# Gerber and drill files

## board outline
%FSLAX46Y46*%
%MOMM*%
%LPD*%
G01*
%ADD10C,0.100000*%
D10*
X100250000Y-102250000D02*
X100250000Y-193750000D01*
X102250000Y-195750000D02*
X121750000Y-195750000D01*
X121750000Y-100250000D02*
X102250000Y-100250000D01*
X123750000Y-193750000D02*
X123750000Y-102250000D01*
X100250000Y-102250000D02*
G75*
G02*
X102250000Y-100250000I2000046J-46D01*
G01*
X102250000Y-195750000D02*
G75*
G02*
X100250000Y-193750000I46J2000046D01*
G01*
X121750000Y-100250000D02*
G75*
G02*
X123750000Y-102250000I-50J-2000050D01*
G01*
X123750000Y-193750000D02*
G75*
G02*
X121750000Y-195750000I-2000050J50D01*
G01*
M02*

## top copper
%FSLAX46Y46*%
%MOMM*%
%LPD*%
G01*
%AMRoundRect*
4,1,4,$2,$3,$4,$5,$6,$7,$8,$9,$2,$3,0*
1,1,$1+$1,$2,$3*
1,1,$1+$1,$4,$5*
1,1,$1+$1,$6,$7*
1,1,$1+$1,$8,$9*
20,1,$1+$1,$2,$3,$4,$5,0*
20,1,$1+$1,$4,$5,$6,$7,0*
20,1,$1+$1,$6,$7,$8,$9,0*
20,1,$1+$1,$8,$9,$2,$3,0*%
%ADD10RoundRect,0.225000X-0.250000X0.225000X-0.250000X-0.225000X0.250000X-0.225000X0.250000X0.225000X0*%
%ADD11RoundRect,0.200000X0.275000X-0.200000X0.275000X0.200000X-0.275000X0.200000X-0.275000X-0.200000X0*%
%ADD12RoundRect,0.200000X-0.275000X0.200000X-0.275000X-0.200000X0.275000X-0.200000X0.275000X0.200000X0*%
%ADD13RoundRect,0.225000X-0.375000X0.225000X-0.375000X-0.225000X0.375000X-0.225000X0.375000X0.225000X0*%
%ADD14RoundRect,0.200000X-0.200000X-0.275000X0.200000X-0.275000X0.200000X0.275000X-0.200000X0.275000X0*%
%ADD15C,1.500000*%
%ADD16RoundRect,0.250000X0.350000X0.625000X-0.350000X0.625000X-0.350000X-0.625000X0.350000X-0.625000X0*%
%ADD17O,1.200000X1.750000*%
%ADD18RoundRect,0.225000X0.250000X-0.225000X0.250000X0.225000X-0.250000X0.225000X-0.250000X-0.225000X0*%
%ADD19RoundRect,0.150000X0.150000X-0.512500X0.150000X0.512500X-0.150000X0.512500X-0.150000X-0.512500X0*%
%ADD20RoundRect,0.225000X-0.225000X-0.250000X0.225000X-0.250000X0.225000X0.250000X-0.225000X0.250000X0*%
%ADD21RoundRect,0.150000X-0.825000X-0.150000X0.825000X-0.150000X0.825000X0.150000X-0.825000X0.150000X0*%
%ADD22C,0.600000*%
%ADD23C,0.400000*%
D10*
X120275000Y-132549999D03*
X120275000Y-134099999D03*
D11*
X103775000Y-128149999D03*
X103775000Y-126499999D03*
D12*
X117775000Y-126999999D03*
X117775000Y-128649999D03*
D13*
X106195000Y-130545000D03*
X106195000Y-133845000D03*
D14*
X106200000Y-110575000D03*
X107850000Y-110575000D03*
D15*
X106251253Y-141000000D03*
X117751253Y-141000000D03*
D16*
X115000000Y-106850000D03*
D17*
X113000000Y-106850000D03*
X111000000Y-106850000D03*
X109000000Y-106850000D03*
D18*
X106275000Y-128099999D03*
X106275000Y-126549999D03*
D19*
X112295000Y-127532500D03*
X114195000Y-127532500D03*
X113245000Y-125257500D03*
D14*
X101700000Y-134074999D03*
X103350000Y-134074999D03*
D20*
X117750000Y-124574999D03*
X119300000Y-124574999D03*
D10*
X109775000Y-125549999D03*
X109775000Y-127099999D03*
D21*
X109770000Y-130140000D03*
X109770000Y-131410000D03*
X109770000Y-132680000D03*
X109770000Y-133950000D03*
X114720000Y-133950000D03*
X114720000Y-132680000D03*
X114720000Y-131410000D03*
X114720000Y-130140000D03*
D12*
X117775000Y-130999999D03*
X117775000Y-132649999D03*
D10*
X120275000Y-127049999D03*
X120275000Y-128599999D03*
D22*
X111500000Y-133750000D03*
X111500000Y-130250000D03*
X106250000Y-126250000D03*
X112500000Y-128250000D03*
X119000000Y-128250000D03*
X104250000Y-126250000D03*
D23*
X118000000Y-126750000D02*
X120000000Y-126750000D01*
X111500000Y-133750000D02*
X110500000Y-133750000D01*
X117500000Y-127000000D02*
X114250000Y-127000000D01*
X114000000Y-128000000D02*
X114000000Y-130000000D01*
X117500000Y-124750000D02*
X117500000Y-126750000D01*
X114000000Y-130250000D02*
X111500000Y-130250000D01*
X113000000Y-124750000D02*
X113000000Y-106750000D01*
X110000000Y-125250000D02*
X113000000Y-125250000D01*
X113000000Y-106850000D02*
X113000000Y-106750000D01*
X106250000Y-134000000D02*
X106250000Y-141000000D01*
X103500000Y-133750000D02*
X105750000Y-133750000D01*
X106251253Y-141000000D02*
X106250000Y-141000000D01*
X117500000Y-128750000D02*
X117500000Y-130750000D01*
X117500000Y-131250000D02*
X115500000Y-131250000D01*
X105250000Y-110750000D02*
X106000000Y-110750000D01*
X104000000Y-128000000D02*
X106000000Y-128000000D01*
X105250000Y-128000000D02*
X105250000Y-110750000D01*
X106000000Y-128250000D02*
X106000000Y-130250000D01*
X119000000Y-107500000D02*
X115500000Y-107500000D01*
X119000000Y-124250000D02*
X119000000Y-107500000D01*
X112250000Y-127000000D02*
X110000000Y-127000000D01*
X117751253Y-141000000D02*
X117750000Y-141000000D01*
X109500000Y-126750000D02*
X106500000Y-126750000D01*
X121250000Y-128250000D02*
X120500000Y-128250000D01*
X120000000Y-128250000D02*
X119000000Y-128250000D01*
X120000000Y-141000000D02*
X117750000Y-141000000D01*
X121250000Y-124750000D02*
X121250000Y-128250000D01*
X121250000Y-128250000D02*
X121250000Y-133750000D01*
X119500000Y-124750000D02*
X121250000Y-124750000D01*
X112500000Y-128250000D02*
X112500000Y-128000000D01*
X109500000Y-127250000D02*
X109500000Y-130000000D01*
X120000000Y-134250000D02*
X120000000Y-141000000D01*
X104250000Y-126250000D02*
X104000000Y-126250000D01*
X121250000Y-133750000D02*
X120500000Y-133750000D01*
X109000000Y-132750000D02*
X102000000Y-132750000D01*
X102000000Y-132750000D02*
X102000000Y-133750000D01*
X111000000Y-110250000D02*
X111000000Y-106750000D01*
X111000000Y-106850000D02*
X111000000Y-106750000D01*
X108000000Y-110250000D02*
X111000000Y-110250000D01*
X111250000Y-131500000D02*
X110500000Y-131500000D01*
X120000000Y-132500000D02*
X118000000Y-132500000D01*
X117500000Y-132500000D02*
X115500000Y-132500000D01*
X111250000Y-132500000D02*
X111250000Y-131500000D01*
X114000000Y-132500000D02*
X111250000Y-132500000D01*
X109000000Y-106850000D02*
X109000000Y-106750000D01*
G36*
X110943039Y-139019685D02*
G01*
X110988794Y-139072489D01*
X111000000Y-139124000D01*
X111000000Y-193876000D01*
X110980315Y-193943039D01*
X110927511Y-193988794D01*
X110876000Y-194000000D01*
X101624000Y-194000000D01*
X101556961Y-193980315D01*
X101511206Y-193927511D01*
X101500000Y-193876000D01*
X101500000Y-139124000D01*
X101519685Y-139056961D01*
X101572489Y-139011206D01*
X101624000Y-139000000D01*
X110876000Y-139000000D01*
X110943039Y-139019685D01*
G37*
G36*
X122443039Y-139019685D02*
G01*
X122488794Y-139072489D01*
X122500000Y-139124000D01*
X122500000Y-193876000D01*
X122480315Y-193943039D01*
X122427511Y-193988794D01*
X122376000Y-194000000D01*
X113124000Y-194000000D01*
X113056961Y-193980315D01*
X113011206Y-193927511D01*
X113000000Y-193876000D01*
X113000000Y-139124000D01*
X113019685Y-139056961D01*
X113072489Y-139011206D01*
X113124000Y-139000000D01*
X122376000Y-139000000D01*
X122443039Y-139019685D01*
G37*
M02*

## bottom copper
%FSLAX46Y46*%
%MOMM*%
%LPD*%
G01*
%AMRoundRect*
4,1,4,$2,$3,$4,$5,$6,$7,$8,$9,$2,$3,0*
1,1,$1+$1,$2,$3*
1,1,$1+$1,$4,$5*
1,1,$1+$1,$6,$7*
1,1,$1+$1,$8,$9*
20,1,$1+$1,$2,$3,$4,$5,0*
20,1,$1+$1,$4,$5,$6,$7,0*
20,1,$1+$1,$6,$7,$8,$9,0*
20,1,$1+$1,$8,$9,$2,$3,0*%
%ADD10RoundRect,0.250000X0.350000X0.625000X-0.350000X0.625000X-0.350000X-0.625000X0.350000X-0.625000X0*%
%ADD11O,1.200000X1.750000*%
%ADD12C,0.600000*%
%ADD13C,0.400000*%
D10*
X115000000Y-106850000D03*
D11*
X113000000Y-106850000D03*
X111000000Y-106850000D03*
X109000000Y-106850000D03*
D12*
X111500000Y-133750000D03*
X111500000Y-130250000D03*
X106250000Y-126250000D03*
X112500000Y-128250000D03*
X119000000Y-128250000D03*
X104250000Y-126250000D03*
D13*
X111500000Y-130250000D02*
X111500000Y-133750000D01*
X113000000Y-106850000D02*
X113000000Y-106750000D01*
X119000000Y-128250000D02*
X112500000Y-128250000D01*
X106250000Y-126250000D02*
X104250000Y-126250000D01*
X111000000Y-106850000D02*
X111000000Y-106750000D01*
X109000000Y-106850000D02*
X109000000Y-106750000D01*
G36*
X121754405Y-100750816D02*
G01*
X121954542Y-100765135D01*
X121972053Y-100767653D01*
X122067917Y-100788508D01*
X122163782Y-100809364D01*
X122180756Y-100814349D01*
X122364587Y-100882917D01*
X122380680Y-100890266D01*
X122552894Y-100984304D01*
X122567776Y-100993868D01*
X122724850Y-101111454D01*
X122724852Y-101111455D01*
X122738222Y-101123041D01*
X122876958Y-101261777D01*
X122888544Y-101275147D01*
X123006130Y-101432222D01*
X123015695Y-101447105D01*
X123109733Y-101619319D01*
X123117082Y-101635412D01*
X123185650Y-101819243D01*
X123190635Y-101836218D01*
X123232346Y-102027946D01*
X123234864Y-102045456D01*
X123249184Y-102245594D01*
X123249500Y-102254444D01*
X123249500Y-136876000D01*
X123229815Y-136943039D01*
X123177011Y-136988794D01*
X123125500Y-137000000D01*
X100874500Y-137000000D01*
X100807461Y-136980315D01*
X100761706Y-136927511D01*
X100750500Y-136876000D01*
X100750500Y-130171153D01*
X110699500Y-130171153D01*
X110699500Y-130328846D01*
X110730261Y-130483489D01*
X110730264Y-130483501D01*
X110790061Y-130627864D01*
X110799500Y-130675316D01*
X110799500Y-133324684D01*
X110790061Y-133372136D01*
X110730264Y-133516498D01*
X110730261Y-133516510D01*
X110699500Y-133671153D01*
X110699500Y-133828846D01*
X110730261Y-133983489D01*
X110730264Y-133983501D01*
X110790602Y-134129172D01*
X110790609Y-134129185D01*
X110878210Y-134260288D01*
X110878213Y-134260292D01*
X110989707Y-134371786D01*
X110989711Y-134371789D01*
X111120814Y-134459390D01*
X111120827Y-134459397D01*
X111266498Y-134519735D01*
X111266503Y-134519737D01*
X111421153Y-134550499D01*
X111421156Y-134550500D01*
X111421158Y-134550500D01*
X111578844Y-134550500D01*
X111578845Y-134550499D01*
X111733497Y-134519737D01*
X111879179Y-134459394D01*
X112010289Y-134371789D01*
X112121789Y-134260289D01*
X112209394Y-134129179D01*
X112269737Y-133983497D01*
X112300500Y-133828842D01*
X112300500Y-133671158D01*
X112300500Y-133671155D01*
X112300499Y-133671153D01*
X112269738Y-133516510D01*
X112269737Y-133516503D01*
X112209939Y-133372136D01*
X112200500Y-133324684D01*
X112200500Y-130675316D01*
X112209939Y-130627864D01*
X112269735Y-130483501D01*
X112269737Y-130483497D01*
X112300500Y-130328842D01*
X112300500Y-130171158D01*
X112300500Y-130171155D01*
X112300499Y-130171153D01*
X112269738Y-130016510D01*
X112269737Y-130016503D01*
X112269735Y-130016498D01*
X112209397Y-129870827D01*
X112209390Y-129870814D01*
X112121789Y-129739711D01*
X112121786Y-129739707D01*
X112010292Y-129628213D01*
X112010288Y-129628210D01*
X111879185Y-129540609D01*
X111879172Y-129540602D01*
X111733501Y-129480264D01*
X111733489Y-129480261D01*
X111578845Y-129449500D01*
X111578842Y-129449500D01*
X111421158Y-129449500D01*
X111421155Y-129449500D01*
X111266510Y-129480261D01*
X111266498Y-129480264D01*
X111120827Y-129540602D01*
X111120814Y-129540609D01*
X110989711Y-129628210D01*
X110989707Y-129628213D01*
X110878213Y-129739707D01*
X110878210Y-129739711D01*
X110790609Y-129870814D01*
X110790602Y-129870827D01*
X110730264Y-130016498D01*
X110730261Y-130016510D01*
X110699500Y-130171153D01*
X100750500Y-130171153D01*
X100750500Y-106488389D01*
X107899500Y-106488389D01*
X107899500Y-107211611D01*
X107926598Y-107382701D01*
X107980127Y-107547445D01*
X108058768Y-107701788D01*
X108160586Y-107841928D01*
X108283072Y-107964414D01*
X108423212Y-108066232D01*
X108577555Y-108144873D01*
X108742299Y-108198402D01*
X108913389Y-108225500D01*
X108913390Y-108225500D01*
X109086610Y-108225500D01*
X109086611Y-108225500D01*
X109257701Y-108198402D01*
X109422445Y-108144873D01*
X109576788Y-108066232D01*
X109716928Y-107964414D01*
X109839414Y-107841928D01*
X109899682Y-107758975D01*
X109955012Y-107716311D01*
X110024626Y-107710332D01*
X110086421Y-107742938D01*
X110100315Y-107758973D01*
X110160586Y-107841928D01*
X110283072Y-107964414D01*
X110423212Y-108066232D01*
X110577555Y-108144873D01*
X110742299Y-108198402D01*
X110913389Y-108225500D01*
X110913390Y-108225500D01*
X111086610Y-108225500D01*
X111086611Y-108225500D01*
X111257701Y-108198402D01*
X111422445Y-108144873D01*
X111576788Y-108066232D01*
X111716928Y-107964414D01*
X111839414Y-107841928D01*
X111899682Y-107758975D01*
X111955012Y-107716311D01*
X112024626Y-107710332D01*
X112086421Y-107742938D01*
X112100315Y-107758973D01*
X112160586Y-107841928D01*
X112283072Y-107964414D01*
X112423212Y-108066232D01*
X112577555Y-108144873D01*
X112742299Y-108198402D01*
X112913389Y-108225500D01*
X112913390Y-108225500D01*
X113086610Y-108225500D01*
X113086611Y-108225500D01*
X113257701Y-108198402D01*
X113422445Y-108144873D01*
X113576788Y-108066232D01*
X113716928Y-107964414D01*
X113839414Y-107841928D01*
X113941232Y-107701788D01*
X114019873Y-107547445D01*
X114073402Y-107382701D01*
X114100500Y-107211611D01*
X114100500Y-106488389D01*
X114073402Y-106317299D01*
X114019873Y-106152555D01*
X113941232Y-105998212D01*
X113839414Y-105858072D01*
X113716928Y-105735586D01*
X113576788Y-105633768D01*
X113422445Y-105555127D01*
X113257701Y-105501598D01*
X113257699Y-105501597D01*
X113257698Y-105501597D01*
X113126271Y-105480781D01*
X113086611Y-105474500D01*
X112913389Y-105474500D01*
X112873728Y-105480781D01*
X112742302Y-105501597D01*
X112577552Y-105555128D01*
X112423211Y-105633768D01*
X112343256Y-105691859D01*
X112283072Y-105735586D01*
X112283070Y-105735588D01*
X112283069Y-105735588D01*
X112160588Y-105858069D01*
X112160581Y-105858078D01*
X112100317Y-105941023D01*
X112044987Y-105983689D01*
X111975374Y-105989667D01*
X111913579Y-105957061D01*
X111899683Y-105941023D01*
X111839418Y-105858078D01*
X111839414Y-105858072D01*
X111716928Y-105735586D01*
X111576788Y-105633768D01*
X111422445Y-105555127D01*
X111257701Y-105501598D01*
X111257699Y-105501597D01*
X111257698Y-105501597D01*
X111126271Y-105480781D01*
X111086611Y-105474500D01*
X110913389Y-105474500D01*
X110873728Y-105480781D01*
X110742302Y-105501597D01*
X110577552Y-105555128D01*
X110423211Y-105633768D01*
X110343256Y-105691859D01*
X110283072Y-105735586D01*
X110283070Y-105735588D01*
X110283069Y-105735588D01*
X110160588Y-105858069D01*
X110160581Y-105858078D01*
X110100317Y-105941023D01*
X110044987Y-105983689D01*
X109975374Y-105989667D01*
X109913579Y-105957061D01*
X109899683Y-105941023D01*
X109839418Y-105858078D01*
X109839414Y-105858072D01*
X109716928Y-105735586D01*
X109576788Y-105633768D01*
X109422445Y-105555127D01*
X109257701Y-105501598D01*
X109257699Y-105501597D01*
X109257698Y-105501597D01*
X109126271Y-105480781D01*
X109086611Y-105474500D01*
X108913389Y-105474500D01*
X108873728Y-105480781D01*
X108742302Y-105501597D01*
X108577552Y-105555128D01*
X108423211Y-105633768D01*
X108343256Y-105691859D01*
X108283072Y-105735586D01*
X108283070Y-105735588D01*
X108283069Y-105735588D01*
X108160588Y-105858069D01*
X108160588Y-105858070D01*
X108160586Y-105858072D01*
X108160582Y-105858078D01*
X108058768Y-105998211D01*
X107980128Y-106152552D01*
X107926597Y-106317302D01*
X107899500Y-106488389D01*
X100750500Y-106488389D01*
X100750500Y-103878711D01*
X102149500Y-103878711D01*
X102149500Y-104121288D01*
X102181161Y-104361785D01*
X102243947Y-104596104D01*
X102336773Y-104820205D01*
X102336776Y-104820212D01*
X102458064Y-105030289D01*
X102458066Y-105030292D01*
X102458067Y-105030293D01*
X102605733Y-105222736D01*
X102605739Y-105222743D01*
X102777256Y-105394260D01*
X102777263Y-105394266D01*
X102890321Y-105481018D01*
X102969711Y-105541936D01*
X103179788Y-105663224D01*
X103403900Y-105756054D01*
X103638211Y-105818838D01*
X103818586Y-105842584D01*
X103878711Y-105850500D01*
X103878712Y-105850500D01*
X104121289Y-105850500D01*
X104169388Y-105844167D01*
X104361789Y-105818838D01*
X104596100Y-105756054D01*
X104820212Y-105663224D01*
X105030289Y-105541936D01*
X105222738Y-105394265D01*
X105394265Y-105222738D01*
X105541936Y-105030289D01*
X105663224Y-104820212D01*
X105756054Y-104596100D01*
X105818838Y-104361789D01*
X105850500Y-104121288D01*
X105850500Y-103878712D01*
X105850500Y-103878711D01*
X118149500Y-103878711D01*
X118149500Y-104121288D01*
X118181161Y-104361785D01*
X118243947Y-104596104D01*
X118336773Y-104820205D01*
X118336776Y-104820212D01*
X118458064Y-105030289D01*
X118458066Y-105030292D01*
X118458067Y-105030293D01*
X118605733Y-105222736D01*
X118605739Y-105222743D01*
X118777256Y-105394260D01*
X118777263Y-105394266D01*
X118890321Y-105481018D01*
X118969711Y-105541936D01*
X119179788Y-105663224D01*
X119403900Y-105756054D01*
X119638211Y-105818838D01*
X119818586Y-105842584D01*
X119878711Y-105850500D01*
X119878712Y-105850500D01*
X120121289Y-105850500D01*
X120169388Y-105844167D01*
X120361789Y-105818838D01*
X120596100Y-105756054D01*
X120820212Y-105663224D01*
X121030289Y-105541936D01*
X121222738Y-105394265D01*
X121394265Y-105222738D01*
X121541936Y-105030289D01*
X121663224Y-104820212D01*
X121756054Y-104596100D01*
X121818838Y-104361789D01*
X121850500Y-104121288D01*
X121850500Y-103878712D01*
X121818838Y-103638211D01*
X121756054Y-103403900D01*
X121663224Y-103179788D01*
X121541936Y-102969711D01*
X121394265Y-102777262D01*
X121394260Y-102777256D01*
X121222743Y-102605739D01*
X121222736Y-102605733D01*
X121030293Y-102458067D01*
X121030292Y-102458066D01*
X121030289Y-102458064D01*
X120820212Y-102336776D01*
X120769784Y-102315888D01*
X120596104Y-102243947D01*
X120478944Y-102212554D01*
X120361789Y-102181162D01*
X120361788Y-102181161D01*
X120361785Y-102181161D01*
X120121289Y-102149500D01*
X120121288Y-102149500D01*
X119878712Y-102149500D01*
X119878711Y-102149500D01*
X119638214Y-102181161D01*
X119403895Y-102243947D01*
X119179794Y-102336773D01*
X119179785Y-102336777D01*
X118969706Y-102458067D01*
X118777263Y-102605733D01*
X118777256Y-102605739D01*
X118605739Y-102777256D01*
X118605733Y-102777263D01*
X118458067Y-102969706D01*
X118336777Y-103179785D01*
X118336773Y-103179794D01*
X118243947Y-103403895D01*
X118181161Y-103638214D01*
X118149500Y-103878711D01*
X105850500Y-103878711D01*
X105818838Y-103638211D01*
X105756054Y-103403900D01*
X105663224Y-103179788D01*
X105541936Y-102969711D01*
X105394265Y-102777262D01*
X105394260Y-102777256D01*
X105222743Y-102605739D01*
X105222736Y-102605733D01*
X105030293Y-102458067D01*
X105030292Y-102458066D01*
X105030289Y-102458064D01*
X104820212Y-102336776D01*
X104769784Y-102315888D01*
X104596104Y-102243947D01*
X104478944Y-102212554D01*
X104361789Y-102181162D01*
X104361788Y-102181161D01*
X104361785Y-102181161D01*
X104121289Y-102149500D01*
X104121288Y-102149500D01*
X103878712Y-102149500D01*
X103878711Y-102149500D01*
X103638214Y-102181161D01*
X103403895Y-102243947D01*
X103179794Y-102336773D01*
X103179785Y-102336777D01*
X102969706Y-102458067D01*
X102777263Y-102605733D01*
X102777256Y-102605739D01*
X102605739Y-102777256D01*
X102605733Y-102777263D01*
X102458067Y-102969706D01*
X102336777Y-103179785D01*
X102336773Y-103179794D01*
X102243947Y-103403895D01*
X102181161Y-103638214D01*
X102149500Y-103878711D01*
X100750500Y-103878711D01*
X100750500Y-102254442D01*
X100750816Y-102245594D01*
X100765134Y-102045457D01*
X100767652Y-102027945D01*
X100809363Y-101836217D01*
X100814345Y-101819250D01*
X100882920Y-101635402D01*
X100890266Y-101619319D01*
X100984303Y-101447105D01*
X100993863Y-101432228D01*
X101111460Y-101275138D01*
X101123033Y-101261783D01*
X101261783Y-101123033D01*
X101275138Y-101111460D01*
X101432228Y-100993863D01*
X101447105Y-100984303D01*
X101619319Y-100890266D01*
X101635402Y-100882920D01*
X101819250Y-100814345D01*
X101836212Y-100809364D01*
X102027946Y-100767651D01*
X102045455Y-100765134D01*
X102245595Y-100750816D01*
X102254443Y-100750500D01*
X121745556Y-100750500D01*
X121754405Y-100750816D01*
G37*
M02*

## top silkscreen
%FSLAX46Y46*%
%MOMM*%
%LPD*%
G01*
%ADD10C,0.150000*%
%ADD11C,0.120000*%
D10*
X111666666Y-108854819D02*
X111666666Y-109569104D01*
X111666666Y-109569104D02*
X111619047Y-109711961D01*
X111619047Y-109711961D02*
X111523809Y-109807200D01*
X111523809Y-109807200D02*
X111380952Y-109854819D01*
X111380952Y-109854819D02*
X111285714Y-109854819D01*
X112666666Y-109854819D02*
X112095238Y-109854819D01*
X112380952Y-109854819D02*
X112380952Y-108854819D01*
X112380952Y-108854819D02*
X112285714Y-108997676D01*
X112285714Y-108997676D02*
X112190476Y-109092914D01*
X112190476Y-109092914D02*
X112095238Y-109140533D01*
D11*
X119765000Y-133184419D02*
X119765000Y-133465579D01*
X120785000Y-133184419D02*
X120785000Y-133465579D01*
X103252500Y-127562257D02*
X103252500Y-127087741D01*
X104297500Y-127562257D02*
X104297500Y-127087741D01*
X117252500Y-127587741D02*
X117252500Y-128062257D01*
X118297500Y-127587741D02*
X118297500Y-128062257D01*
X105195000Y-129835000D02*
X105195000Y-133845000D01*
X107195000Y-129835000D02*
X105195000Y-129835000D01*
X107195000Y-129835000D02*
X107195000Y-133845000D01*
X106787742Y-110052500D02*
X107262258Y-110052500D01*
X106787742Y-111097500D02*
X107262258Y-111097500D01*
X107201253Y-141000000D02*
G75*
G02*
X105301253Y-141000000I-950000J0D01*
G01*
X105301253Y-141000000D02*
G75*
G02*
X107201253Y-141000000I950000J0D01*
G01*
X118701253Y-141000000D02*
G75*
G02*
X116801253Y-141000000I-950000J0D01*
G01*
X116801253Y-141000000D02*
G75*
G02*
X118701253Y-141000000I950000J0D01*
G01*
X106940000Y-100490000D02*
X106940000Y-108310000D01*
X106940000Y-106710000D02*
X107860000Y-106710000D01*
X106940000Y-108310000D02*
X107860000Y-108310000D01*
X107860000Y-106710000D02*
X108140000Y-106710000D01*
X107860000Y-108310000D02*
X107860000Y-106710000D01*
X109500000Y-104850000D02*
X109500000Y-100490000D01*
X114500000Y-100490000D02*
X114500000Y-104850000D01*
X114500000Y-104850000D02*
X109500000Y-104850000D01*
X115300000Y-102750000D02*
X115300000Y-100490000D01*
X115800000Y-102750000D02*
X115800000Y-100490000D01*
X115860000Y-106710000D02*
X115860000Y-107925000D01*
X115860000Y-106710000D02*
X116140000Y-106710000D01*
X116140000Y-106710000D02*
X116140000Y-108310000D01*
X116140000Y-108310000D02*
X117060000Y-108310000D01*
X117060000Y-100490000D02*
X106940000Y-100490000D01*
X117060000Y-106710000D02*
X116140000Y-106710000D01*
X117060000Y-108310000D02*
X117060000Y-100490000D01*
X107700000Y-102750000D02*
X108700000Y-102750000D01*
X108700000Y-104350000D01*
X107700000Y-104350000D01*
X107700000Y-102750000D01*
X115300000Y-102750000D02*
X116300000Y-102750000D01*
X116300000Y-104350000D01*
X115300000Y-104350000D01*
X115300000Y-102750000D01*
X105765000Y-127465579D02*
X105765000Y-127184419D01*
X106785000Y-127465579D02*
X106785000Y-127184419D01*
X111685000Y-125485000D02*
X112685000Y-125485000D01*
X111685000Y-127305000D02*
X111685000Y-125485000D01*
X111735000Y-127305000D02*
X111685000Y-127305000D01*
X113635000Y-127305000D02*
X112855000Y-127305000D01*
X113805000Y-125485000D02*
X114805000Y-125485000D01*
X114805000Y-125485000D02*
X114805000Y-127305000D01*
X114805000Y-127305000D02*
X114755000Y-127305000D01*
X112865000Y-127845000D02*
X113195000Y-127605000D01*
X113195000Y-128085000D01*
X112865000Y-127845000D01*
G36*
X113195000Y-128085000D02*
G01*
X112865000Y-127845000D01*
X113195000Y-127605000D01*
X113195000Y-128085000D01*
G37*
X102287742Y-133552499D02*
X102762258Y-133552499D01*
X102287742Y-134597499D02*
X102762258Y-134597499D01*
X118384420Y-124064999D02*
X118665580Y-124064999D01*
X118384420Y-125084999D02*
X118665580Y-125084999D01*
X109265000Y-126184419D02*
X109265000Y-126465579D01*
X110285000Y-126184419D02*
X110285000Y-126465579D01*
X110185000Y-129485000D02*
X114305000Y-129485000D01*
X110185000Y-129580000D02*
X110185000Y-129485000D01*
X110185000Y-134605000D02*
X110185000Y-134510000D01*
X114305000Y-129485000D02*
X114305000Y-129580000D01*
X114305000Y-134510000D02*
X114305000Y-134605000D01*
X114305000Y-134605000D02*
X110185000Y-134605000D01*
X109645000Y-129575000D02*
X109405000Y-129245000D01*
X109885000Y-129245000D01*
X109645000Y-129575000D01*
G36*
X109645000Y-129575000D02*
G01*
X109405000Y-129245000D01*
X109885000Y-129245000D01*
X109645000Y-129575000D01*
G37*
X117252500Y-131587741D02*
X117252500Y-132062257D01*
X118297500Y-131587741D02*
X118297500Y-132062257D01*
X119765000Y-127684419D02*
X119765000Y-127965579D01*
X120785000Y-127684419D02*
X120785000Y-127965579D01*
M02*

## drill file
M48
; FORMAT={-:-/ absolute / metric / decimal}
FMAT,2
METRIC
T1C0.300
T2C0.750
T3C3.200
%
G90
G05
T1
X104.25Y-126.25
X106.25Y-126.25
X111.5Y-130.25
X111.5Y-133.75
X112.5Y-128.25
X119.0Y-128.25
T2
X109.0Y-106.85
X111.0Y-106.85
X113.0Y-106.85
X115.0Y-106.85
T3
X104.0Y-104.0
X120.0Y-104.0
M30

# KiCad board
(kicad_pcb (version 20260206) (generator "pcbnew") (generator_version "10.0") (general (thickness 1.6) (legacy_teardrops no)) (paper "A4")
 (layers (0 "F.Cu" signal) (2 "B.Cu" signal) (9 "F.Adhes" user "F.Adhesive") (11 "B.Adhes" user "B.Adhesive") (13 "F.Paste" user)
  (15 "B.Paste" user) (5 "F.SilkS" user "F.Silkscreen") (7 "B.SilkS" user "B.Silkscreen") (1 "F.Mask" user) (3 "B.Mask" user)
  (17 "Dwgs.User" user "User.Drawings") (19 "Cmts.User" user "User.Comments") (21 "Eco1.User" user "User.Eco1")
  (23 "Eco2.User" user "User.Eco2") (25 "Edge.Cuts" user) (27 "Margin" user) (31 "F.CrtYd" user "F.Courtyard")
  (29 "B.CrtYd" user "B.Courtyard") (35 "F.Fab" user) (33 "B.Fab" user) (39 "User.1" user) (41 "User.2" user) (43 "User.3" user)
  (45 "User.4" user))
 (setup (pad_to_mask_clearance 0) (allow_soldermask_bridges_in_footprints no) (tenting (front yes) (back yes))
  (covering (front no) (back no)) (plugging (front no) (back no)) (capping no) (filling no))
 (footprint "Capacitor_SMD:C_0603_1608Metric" (layer "F.Cu") (at 120.275 133.324999 -90)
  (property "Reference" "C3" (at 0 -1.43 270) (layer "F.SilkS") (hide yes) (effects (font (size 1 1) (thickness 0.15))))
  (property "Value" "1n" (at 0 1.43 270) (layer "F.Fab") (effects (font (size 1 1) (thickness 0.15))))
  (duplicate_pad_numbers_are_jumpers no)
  (fp_line (start -0.14058 0.51) (end 0.14058 0.51) (stroke (width 0.12) (type solid)) (layer "F.SilkS"))
  (fp_line (start -0.14058 -0.51) (end 0.14058 -0.51) (stroke (width 0.12) (type solid)) (layer "F.SilkS"))
  (pad "1" smd roundrect (at -0.775 0 270) (size 0.9 0.95) (layers "F.Cu" "F.Mask" "F.Paste") (roundrect_rratio 0.25) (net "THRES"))
  (pad "2" smd roundrect (at 0.775 0 270) (size 0.9 0.95) (layers "F.Cu" "F.Mask" "F.Paste") (roundrect_rratio 0.25) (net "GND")))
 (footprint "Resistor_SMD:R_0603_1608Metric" (layer "F.Cu") (at 103.775 127.324999 90)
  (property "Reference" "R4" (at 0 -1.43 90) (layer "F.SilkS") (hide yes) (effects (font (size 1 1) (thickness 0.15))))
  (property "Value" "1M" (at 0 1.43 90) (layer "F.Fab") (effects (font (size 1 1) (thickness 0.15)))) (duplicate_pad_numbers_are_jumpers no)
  (fp_line (start -0.237258 -0.5225) (end 0.237258 -0.5225) (stroke (width 0.12) (type solid)) (layer "F.SilkS"))
  (fp_line (start -0.237258 0.5225) (end 0.237258 0.5225) (stroke (width 0.12) (type solid)) (layer "F.SilkS"))
  (pad "1" smd roundrect (at -0.825 0 90) (size 0.8 0.95) (layers "F.Cu" "F.Mask" "F.Paste") (roundrect_rratio 0.25) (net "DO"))
  (pad "2" smd roundrect (at 0.825 0 90) (size 0.8 0.95) (layers "F.Cu" "F.Mask" "F.Paste") (roundrect_rratio 0.25) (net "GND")))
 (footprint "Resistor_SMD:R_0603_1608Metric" (layer "F.Cu") (at 117.775 127.824999 -90)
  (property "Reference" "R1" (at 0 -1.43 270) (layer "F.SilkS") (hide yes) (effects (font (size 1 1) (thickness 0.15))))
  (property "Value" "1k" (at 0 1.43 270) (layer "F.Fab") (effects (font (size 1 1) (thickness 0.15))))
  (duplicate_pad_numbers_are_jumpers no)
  (fp_line (start -0.237258 0.5225) (end 0.237258 0.5225) (stroke (width 0.12) (type solid)) (layer "F.SilkS"))
  (fp_line (start -0.237258 -0.5225) (end 0.237258 -0.5225) (stroke (width 0.12) (type solid)) (layer "F.SilkS"))
  (pad "1" smd roundrect (at -0.825 0 270) (size 0.8 0.95) (layers "F.Cu" "F.Mask" "F.Paste") (roundrect_rratio 0.25) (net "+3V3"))
  (pad "2" smd roundrect (at 0.825 0 270) (size 0.8 0.95) (layers "F.Cu" "F.Mask" "F.Paste") (roundrect_rratio 0.25) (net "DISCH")))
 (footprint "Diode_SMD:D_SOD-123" (layer "F.Cu") (at 106.195 132.195 -90)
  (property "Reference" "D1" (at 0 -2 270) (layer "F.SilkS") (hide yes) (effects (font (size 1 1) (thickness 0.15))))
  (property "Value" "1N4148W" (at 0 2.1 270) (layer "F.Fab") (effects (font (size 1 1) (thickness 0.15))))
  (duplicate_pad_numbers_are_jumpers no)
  (fp_line (start -2.36 1) (end 1.65 1) (stroke (width 0.12) (type solid)) (layer "F.SilkS"))
  (fp_line (start -2.36 -1) (end -2.36 1) (stroke (width 0.12) (type solid)) (layer "F.SilkS"))
  (fp_line (start -2.36 -1) (end 1.65 -1) (stroke (width 0.12) (type solid)) (layer "F.SilkS"))
  (pad "1" smd roundrect (at -1.65 0 270) (size 0.9 1.2) (layers "F.Cu" "F.Mask" "F.Paste") (roundrect_rratio 0.25) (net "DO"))
  (pad "2" smd roundrect (at 1.65 0 270) (size 0.9 1.2) (layers "F.Cu" "F.Mask" "F.Paste") (roundrect_rratio 0.25) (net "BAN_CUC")))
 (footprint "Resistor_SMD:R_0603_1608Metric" (layer "F.Cu") (at 107.025 110.575)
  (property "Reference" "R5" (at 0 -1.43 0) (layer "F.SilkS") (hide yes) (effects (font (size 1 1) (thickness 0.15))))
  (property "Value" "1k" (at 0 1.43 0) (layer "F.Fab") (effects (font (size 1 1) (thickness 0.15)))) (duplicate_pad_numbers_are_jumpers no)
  (fp_line (start -0.237258 -0.5225) (end 0.237258 -0.5225) (stroke (width 0.12) (type solid)) (layer "F.SilkS"))
  (fp_line (start -0.237258 0.5225) (end 0.237258 0.5225) (stroke (width 0.12) (type solid)) (layer "F.SilkS"))
  (pad "1" smd roundrect (at -0.825 0) (size 0.8 0.95) (layers "F.Cu" "F.Mask" "F.Paste") (roundrect_rratio 0.25) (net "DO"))
  (pad "2" smd roundrect (at 0.825 0) (size 0.8 0.95) (layers "F.Cu" "F.Mask" "F.Paste") (roundrect_rratio 0.25) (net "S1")))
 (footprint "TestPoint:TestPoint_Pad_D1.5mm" (layer "F.Cu") (at 106.251253 141)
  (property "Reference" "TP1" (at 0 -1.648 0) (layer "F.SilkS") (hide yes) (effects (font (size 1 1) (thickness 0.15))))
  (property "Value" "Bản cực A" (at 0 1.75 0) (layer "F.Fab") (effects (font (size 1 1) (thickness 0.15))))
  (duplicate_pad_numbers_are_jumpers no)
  (fp_circle (center 0 0) (end 0 0.95) (stroke (width 0.12) (type solid)) (fill no) (layer "F.SilkS"))
  (pad "1" smd circle (at 0 0) (size 1.5 1.5) (layers "F.Cu" "F.Mask") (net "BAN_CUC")))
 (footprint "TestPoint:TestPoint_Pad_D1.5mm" (layer "F.Cu") (at 117.751253 141)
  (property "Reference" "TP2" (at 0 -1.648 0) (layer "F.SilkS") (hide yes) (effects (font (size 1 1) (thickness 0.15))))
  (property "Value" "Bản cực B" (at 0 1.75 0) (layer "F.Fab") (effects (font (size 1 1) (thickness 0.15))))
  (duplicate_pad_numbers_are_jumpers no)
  (fp_circle (center 0 0) (end 0 0.95) (stroke (width 0.12) (type solid)) (fill no) (layer "F.SilkS"))
  (pad "1" smd circle (at 0 0) (size 1.5 1.5) (layers "F.Cu" "F.Mask") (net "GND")))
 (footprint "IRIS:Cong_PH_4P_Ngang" (layer "F.Cu") (at 115 106.85 180)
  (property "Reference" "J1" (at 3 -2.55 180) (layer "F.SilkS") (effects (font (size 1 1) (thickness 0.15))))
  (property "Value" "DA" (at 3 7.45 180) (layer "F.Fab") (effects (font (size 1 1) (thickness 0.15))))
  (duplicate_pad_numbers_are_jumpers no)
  (fp_line (start 8.06 6.36) (end 8.06 -1.46) (stroke (width 0.12) (type solid)) (layer "F.SilkS"))
  (fp_line (start 8.06 0.14) (end 7.14 0.14) (stroke (width 0.12) (type solid)) (layer "F.SilkS"))
  (fp_line (start 8.06 -1.46) (end 7.14 -1.46) (stroke (width 0.12) (type solid)) (layer "F.SilkS"))
  (fp_line (start 7.14 0.14) (end 6.86 0.14) (stroke (width 0.12) (type solid)) (layer "F.SilkS"))
  (fp_line (start 7.14 -1.46) (end 7.14 0.14) (stroke (width 0.12) (type solid)) (layer "F.SilkS"))
  (fp_line (start 5.5 2) (end 5.5 6.36) (stroke (width 0.12) (type solid)) (layer "F.SilkS"))
  (fp_line (start 0.5 6.36) (end 0.5 2) (stroke (width 0.12) (type solid)) (layer "F.SilkS"))
  (fp_line (start 0.5 2) (end 5.5 2) (stroke (width 0.12) (type solid)) (layer "F.SilkS"))
  (fp_line (start -0.3 4.1) (end -0.3 6.36) (stroke (width 0.12) (type solid)) (layer "F.SilkS"))
  (fp_line (start -0.8 4.1) (end -0.8 6.36) (stroke (width 0.12) (type solid)) (layer "F.SilkS"))
  (fp_line (start -0.86 0.14) (end -0.86 -1.075) (stroke (width 0.12) (type solid)) (layer "F.SilkS"))
  (fp_line (start -0.86 0.14) (end -1.14 0.14) (stroke (width 0.12) (type solid)) (layer "F.SilkS"))
  (fp_line (start -1.14 0.14) (end -1.14 -1.46) (stroke (width 0.12) (type solid)) (layer "F.SilkS"))
  (fp_line (start -1.14 -1.46) (end -2.06 -1.46) (stroke (width 0.12) (type solid)) (layer "F.SilkS"))
  (fp_line (start -2.06 6.36) (end 8.06 6.36) (stroke (width 0.12) (type solid)) (layer "F.SilkS"))
  (fp_line (start -2.06 0.14) (end -1.14 0.14) (stroke (width 0.12) (type solid)) (layer "F.SilkS"))
  (fp_line (start -2.06 -1.46) (end -2.06 6.36) (stroke (width 0.12) (type solid)) (layer "F.SilkS"))
  (fp_rect (start 6.3 2.5) (end 7.3 4.1) (stroke (width 0.12) (type solid)) (fill no) (layer "F.SilkS"))
  (fp_rect (start -1.3 2.5) (end -0.3 4.1) (stroke (width 0.12) (type solid)) (fill no) (layer "F.SilkS"))
  (pad "1" thru_hole roundrect (at 0 0 180) (size 1.2 1.75) (drill 0.75) (layers "*.Cu" "*.Mask") (remove_unused_layers no)
   (roundrect_rratio 0.208333) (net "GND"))
  (pad "2" thru_hole oval (at 2 0 180) (size 1.2 1.75) (drill 0.75) (layers "*.Cu" "*.Mask") (remove_unused_layers no) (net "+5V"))
  (pad "3" thru_hole oval (at 4 0 180) (size 1.2 1.75) (drill 0.75) (layers "*.Cu" "*.Mask") (remove_unused_layers no) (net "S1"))
  (pad "4" thru_hole oval (at 6 0 180) (size 1.2 1.75) (drill 0.75) (layers "*.Cu" "*.Mask") (remove_unused_layers no)
   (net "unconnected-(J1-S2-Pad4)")))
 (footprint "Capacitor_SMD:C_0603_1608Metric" (layer "F.Cu") (at 106.275 127.324999 90)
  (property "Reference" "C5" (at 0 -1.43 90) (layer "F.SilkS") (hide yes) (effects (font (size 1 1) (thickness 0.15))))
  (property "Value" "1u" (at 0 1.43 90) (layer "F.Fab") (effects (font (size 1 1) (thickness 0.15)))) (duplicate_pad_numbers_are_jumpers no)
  (fp_line (start -0.14058 -0.51) (end 0.14058 -0.51) (stroke (width 0.12) (type solid)) (layer "F.SilkS"))
  (fp_line (start -0.14058 0.51) (end 0.14058 0.51) (stroke (width 0.12) (type solid)) (layer "F.SilkS"))
  (pad "1" smd roundrect (at -0.775 0 90) (size 0.9 0.95) (layers "F.Cu" "F.Mask" "F.Paste") (roundrect_rratio 0.25) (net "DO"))
  (pad "2" smd roundrect (at 0.775 0 90) (size 0.9 0.95) (layers "F.Cu" "F.Mask" "F.Paste") (roundrect_rratio 0.25) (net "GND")))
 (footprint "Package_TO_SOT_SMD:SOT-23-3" (layer "F.Cu") (at 113.245 126.395 90)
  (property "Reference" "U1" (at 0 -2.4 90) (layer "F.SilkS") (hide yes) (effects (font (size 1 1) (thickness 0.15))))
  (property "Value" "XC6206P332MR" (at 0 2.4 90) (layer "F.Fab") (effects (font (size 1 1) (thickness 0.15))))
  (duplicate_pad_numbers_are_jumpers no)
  (fp_line (start 0.91 -1.56) (end 0.91 -0.56) (stroke (width 0.12) (type solid)) (layer "F.SilkS"))
  (fp_line (start -0.91 -1.56) (end 0.91 -1.56) (stroke (width 0.12) (type solid)) (layer "F.SilkS"))
  (fp_line (start -0.91 -1.51) (end -0.91 -1.56) (stroke (width 0.12) (type solid)) (layer "F.SilkS"))
  (fp_line (start -0.91 0.39) (end -0.91 -0.39) (stroke (width 0.12) (type solid)) (layer "F.SilkS"))
  (fp_line (start 0.91 0.56) (end 0.91 1.56) (stroke (width 0.12) (type solid)) (layer "F.SilkS"))
  (fp_line (start 0.91 1.56) (end -0.91 1.56) (stroke (width 0.12) (type solid)) (layer "F.SilkS"))
  (fp_line (start -0.91 1.56) (end -0.91 1.51) (stroke (width 0.12) (type solid)) (layer "F.SilkS"))
  (fp_poly (pts (xy -1.45 -0.38) (xy -1.21 -0.05) (xy -1.69 -0.05)) (stroke (width 0.12) (type solid)) (fill yes) (layer "F.SilkS"))
  (pad "1" smd roundrect (at -1.1375 -0.95 90) (size 1.325 0.6) (layers "F.Cu" "F.Mask" "F.Paste") (roundrect_rratio 0.25) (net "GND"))
  (pad "2" smd roundrect (at -1.1375 0.95 90) (size 1.325 0.6) (layers "F.Cu" "F.Mask" "F.Paste") (roundrect_rratio 0.25) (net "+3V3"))
  (pad "3" smd roundrect (at 1.1375 0 90) (size 1.325 0.6) (layers "F.Cu" "F.Mask" "F.Paste") (roundrect_rratio 0.25) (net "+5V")))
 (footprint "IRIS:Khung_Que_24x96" (layer "F.Cu") (at 100 196)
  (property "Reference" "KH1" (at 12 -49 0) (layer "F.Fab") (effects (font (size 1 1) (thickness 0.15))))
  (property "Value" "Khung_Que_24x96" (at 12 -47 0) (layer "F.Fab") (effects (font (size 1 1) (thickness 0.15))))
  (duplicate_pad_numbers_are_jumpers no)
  (fp_line (start 0.25 -93.75) (end 0.25 -2.25) (stroke (width 0.1) (type solid)) (layer "Edge.Cuts"))
  (fp_line (start 2.25 -0.25) (end 21.75 -0.25) (stroke (width 0.1) (type solid)) (layer "Edge.Cuts"))
  (fp_line (start 21.75 -95.75) (end 2.25 -95.75) (stroke (width 0.1) (type solid)) (layer "Edge.Cuts"))
  (fp_line (start 23.75 -2.25) (end 23.75 -93.75) (stroke (width 0.1) (type solid)) (layer "Edge.Cuts"))
  (fp_arc (start 0.25 -93.75) (mid 0.8358 -95.1642) (end 2.25 -95.75) (stroke (width 0.1) (type solid)) (layer "Edge.Cuts"))
  (fp_arc (start 2.25 -0.25) (mid 0.8358 -0.8358) (end 0.25 -2.25) (stroke (width 0.1) (type solid)) (layer "Edge.Cuts"))
  (fp_arc (start 21.75 -95.75) (mid 23.164199 -95.164199) (end 23.75 -93.75) (stroke (width 0.1) (type solid)) (layer "Edge.Cuts"))
  (fp_arc (start 23.75 -2.25) (mid 23.164199 -0.835801) (end 21.75 -0.25) (stroke (width 0.1) (type solid)) (layer "Edge.Cuts"))
  (pad "" np_thru_hole circle (at 4 -92) (size 3.2 3.2) (drill 3.2) (layers "*.Cu" "*.Mask"))
  (pad "" np_thru_hole circle (at 20 -92) (size 3.2 3.2) (drill 3.2) (layers "*.Cu" "*.Mask")))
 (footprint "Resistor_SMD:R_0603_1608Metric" (layer "F.Cu") (at 102.525 134.074999)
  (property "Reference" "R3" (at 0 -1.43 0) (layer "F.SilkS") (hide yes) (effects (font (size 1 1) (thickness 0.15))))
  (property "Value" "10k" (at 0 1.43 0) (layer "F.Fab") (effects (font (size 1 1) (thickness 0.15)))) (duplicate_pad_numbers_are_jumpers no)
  (fp_line (start -0.237258 -0.5225) (end 0.237258 -0.5225) (stroke (width 0.12) (type solid)) (layer "F.SilkS"))
  (fp_line (start -0.237258 0.5225) (end 0.237258 0.5225) (stroke (width 0.12) (type solid)) (layer "F.SilkS"))
  (pad "1" smd roundrect (at -0.825 0) (size 0.8 0.95) (layers "F.Cu" "F.Mask" "F.Paste") (roundrect_rratio 0.25) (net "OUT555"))
  (pad "2" smd roundrect (at 0.825 0) (size 0.8 0.95) (layers "F.Cu" "F.Mask" "F.Paste") (roundrect_rratio 0.25) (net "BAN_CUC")))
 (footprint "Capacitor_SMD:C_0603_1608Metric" (layer "F.Cu") (at 118.525 124.574999)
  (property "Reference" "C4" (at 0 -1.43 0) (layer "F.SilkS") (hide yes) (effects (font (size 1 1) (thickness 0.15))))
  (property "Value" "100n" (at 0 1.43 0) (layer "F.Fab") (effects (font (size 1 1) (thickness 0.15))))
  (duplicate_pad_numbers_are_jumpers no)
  (fp_line (start -0.14058 -0.51) (end 0.14058 -0.51) (stroke (width 0.12) (type solid)) (layer "F.SilkS"))
  (fp_line (start -0.14058 0.51) (end 0.14058 0.51) (stroke (width 0.12) (type solid)) (layer "F.SilkS"))
  (pad "1" smd roundrect (at -0.775 0) (size 0.9 0.95) (layers "F.Cu" "F.Mask" "F.Paste") (roundrect_rratio 0.25) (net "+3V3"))
  (pad "2" smd roundrect (at 0.775 0) (size 0.9 0.95) (layers "F.Cu" "F.Mask" "F.Paste") (roundrect_rratio 0.25) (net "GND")))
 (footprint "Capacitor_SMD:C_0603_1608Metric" (layer "F.Cu") (at 109.775 126.324999 -90)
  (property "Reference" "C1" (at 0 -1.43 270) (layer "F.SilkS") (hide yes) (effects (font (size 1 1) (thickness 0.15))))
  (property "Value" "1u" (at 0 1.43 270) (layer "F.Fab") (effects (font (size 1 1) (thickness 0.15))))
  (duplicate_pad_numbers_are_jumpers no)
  (fp_line (start -0.14058 0.51) (end 0.14058 0.51) (stroke (width 0.12) (type solid)) (layer "F.SilkS"))
  (fp_line (start -0.14058 -0.51) (end 0.14058 -0.51) (stroke (width 0.12) (type solid)) (layer "F.SilkS"))
  (pad "1" smd roundrect (at -0.775 0 270) (size 0.9 0.95) (layers "F.Cu" "F.Mask" "F.Paste") (roundrect_rratio 0.25) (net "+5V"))
  (pad "2" smd roundrect (at 0.775 0 270) (size 0.9 0.95) (layers "F.Cu" "F.Mask" "F.Paste") (roundrect_rratio 0.25) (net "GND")))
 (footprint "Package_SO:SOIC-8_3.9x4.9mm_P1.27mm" (layer "F.Cu") (at 112.245 132.045)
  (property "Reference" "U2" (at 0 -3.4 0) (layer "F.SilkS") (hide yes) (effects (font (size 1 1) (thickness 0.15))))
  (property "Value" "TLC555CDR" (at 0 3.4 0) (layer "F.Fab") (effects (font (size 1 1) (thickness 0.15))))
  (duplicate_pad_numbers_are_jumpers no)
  (fp_line (start -2.06 -2.56) (end 2.06 -2.56) (stroke (width 0.12) (type solid)) (layer "F.SilkS"))
  (fp_line (start -2.06 -2.465) (end -2.06 -2.56) (stroke (width 0.12) (type solid)) (layer "F.SilkS"))
  (fp_line (start -2.06 2.56) (end -2.06 2.465) (stroke (width 0.12) (type solid)) (layer "F.SilkS"))
  (fp_line (start 2.06 -2.56) (end 2.06 -2.465) (stroke (width 0.12) (type solid)) (layer "F.SilkS"))
  (fp_line (start 2.06 2.465) (end 2.06 2.56) (stroke (width 0.12) (type solid)) (layer "F.SilkS"))
  (fp_line (start 2.06 2.56) (end -2.06 2.56) (stroke (width 0.12) (type solid)) (layer "F.SilkS"))
  (fp_poly (pts (xy -2.6 -2.47) (xy -2.84 -2.8) (xy -2.36 -2.8)) (stroke (width 0.12) (type solid)) (fill yes) (layer "F.SilkS"))
  (pad "1" smd roundrect (at -2.475 -1.905) (size 1.95 0.6) (layers "F.Cu" "F.Mask" "F.Paste") (roundrect_rratio 0.25) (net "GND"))
  (pad "2" smd roundrect (at -2.475 -0.635) (size 1.95 0.6) (layers "F.Cu" "F.Mask" "F.Paste") (roundrect_rratio 0.25) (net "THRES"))
  (pad "3" smd roundrect (at -2.475 0.635) (size 1.95 0.6) (layers "F.Cu" "F.Mask" "F.Paste") (roundrect_rratio 0.25) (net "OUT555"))
  (pad "4" smd roundrect (at -2.475 1.905) (size 1.95 0.6) (layers "F.Cu" "F.Mask" "F.Paste") (roundrect_rratio 0.25) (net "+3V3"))
  (pad "5" smd roundrect (at 2.475 1.905) (size 1.95 0.6) (layers "F.Cu" "F.Mask" "F.Paste") (roundrect_rratio 0.25)
   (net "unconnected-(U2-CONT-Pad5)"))
  (pad "6" smd roundrect (at 2.475 0.635) (size 1.95 0.6) (layers "F.Cu" "F.Mask" "F.Paste") (roundrect_rratio 0.25) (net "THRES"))
  (pad "7" smd roundrect (at 2.475 -0.635) (size 1.95 0.6) (layers "F.Cu" "F.Mask" "F.Paste") (roundrect_rratio 0.25) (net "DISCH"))
  (pad "8" smd roundrect (at 2.475 -1.905) (size 1.95 0.6) (layers "F.Cu" "F.Mask" "F.Paste") (roundrect_rratio 0.25) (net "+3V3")))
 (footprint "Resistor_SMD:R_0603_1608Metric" (layer "F.Cu") (at 117.775 131.824999 -90)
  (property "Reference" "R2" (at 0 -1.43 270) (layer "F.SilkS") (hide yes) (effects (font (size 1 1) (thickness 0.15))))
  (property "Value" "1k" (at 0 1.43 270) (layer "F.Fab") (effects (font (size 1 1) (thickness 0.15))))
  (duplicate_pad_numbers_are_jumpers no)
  (fp_line (start -0.237258 0.5225) (end 0.237258 0.5225) (stroke (width 0.12) (type solid)) (layer "F.SilkS"))
  (fp_line (start -0.237258 -0.5225) (end 0.237258 -0.5225) (stroke (width 0.12) (type solid)) (layer "F.SilkS"))
  (pad "1" smd roundrect (at -0.825 0 270) (size 0.8 0.95) (layers "F.Cu" "F.Mask" "F.Paste") (roundrect_rratio 0.25) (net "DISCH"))
  (pad "2" smd roundrect (at 0.825 0 270) (size 0.8 0.95) (layers "F.Cu" "F.Mask" "F.Paste") (roundrect_rratio 0.25) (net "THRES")))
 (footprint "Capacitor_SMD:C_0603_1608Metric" (layer "F.Cu") (at 120.275 127.824999 -90)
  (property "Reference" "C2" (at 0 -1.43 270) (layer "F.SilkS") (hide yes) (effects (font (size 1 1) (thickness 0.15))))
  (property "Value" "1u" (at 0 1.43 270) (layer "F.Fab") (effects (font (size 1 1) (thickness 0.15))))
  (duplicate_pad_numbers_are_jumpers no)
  (fp_line (start -0.14058 0.51) (end 0.14058 0.51) (stroke (width 0.12) (type solid)) (layer "F.SilkS"))
  (fp_line (start -0.14058 -0.51) (end 0.14058 -0.51) (stroke (width 0.12) (type solid)) (layer "F.SilkS"))
  (pad "1" smd roundrect (at -0.775 0 270) (size 0.9 0.95) (layers "F.Cu" "F.Mask" "F.Paste") (roundrect_rratio 0.25) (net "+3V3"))
  (pad "2" smd roundrect (at 0.775 0 270) (size 0.9 0.95) (layers "F.Cu" "F.Mask" "F.Paste") (roundrect_rratio 0.25) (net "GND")))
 (segment (start 118 126.75) (end 120 126.75) (width 0.4) (layer "F.Cu") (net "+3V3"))
 (segment (start 111.5 133.75) (end 110.5 133.75) (width 0.4) (layer "F.Cu") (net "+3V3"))
 (segment (start 117.5 127) (end 114.25 127) (width 0.4) (layer "F.Cu") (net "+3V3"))
 (segment (start 114 128) (end 114 130) (width 0.4) (layer "F.Cu") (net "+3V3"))
 (segment (start 117.5 124.75) (end 117.5 126.75) (width 0.4) (layer "F.Cu") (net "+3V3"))
 (segment (start 114 130.25) (end 111.5 130.25) (width 0.4) (layer "F.Cu") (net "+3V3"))
 (via (at 111.5 133.75) (size 0.6) (drill 0.3) (layers "F.Cu" "B.Cu") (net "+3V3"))
 (via (at 111.5 130.25) (size 0.6) (drill 0.3) (layers "F.Cu" "B.Cu") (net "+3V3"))
 (segment (start 111.5 130.25) (end 111.5 133.75) (width 0.4) (layer "B.Cu") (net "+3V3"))
 (segment (start 113 124.75) (end 113 106.75) (width 0.4) (layer "F.Cu") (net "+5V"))
 (segment (start 110 125.25) (end 113 125.25) (width 0.4) (layer "F.Cu") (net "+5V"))
 (segment (start 113 106.85) (end 113 106.75) (width 0.4) (layer "F.Cu") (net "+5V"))
 (segment (start 113 106.85) (end 113 106.75) (width 0.4) (layer "B.Cu") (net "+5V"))
 (segment (start 106.25 134) (end 106.25 141) (width 0.4) (layer "F.Cu") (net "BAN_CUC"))
 (segment (start 103.5 133.75) (end 105.75 133.75) (width 0.4) (layer "F.Cu") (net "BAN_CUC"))
 (segment (start 106.251253 141) (end 106.25 141) (width 0.4) (layer "F.Cu") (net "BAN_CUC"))
 (segment (start 117.5 128.75) (end 117.5 130.75) (width 0.4) (layer "F.Cu") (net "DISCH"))
 (segment (start 117.5 131.25) (end 115.5 131.25) (width 0.4) (layer "F.Cu") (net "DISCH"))
 (segment (start 105.25 110.75) (end 106 110.75) (width 0.4) (layer "F.Cu") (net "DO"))
 (segment (start 104 128) (end 106 128) (width 0.4) (layer "F.Cu") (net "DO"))
 (segment (start 105.25 128) (end 105.25 110.75) (width 0.4) (layer "F.Cu") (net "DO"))
 (segment (start 106 128.25) (end 106 130.25) (width 0.4) (layer "F.Cu") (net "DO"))
 (segment (start 119 107.5) (end 115.5 107.5) (width 0.4) (layer "F.Cu") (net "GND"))
 (segment (start 119 124.25) (end 119 107.5) (width 0.4) (layer "F.Cu") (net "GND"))
 (segment (start 112.25 127) (end 110 127) (width 0.4) (layer "F.Cu") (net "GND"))
 (segment (start 117.751253 141) (end 117.75 141) (width 0.4) (layer "F.Cu") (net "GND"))
 (segment (start 109.5 126.75) (end 106.5 126.75) (width 0.4) (layer "F.Cu") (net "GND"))
 (segment (start 121.25 128.25) (end 120.5 128.25) (width 0.4) (layer "F.Cu") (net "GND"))
 (segment (start 120 128.25) (end 119 128.25) (width 0.4) (layer "F.Cu") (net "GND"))
 (segment (start 120 141) (end 117.75 141) (width 0.4) (layer "F.Cu") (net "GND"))
 (segment (start 121.25 124.75) (end 121.25 128.25) (width 0.4) (layer "F.Cu") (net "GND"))
 (segment (start 121.25 128.25) (end 121.25 133.75) (width 0.4) (layer "F.Cu") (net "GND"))
 (segment (start 119.5 124.75) (end 121.25 124.75) (width 0.4) (layer "F.Cu") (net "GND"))
 (segment (start 112.5 128.25) (end 112.5 128) (width 0.4) (layer "F.Cu") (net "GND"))
 (segment (start 109.5 127.25) (end 109.5 130) (width 0.4) (layer "F.Cu") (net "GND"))
 (segment (start 120 134.25) (end 120 141) (width 0.4) (layer "F.Cu") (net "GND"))
 (segment (start 104.25 126.25) (end 104 126.25) (width 0.4) (layer "F.Cu") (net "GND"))
 (segment (start 121.25 133.75) (end 120.5 133.75) (width 0.4) (layer "F.Cu") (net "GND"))
 (via (at 106.25 126.25) (size 0.6) (drill 0.3) (layers "F.Cu" "B.Cu") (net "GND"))
 (via (at 112.5 128.25) (size 0.6) (drill 0.3) (layers "F.Cu" "B.Cu") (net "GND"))
 (via (at 119 128.25) (size 0.6) (drill 0.3) (layers "F.Cu" "B.Cu") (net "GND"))
 (via (at 104.25 126.25) (size 0.6) (drill 0.3) (layers "F.Cu" "B.Cu") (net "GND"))
 (segment (start 119 128.25) (end 112.5 128.25) (width 0.4) (layer "B.Cu") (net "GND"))
 (segment (start 106.25 126.25) (end 104.25 126.25) (width 0.4) (layer "B.Cu") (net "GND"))
 (segment (start 109 132.75) (end 102 132.75) (width 0.4) (layer "F.Cu") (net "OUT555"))
 (segment (start 102 132.75) (end 102 133.75) (width 0.4) (layer "F.Cu") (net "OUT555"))
 (segment (start 111 110.25) (end 111 106.75) (width 0.4) (layer "F.Cu") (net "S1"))
 (segment (start 111 106.85) (end 111 106.75) (width 0.4) (layer "F.Cu") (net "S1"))
 (segment (start 108 110.25) (end 111 110.25) (width 0.4) (layer "F.Cu") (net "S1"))
 (segment (start 111 106.85) (end 111 106.75) (width 0.4) (layer "B.Cu") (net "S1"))
 (segment (start 111.25 131.5) (end 110.5 131.5) (width 0.4) (layer "F.Cu") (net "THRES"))
 (segment (start 120 132.5) (end 118 132.5) (width 0.4) (layer "F.Cu") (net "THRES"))
 (segment (start 117.5 132.5) (end 115.5 132.5) (width 0.4) (layer "F.Cu") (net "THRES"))
 (segment (start 111.25 132.5) (end 111.25 131.5) (width 0.4) (layer "F.Cu") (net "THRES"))
 (segment (start 114 132.5) (end 111.25 132.5) (width 0.4) (layer "F.Cu") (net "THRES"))
 (segment (start 109 106.85) (end 109 106.75) (width 0.4) (layer "F.Cu") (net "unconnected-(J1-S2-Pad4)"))
 (segment (start 109 106.85) (end 109 106.75) (width 0.4) (layer "B.Cu") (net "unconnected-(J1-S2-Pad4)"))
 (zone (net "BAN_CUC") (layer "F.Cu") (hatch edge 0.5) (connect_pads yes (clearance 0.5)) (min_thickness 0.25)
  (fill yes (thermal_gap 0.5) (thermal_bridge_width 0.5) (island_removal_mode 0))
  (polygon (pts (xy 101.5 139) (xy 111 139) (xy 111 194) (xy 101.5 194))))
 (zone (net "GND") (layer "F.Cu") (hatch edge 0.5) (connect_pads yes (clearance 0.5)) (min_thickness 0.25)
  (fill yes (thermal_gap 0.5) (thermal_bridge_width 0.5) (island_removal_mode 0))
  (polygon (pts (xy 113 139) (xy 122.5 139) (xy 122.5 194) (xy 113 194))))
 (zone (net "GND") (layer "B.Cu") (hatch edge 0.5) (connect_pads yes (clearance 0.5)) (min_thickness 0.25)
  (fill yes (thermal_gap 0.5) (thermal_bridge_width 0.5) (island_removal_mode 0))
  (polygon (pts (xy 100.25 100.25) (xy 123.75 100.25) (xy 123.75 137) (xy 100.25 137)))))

